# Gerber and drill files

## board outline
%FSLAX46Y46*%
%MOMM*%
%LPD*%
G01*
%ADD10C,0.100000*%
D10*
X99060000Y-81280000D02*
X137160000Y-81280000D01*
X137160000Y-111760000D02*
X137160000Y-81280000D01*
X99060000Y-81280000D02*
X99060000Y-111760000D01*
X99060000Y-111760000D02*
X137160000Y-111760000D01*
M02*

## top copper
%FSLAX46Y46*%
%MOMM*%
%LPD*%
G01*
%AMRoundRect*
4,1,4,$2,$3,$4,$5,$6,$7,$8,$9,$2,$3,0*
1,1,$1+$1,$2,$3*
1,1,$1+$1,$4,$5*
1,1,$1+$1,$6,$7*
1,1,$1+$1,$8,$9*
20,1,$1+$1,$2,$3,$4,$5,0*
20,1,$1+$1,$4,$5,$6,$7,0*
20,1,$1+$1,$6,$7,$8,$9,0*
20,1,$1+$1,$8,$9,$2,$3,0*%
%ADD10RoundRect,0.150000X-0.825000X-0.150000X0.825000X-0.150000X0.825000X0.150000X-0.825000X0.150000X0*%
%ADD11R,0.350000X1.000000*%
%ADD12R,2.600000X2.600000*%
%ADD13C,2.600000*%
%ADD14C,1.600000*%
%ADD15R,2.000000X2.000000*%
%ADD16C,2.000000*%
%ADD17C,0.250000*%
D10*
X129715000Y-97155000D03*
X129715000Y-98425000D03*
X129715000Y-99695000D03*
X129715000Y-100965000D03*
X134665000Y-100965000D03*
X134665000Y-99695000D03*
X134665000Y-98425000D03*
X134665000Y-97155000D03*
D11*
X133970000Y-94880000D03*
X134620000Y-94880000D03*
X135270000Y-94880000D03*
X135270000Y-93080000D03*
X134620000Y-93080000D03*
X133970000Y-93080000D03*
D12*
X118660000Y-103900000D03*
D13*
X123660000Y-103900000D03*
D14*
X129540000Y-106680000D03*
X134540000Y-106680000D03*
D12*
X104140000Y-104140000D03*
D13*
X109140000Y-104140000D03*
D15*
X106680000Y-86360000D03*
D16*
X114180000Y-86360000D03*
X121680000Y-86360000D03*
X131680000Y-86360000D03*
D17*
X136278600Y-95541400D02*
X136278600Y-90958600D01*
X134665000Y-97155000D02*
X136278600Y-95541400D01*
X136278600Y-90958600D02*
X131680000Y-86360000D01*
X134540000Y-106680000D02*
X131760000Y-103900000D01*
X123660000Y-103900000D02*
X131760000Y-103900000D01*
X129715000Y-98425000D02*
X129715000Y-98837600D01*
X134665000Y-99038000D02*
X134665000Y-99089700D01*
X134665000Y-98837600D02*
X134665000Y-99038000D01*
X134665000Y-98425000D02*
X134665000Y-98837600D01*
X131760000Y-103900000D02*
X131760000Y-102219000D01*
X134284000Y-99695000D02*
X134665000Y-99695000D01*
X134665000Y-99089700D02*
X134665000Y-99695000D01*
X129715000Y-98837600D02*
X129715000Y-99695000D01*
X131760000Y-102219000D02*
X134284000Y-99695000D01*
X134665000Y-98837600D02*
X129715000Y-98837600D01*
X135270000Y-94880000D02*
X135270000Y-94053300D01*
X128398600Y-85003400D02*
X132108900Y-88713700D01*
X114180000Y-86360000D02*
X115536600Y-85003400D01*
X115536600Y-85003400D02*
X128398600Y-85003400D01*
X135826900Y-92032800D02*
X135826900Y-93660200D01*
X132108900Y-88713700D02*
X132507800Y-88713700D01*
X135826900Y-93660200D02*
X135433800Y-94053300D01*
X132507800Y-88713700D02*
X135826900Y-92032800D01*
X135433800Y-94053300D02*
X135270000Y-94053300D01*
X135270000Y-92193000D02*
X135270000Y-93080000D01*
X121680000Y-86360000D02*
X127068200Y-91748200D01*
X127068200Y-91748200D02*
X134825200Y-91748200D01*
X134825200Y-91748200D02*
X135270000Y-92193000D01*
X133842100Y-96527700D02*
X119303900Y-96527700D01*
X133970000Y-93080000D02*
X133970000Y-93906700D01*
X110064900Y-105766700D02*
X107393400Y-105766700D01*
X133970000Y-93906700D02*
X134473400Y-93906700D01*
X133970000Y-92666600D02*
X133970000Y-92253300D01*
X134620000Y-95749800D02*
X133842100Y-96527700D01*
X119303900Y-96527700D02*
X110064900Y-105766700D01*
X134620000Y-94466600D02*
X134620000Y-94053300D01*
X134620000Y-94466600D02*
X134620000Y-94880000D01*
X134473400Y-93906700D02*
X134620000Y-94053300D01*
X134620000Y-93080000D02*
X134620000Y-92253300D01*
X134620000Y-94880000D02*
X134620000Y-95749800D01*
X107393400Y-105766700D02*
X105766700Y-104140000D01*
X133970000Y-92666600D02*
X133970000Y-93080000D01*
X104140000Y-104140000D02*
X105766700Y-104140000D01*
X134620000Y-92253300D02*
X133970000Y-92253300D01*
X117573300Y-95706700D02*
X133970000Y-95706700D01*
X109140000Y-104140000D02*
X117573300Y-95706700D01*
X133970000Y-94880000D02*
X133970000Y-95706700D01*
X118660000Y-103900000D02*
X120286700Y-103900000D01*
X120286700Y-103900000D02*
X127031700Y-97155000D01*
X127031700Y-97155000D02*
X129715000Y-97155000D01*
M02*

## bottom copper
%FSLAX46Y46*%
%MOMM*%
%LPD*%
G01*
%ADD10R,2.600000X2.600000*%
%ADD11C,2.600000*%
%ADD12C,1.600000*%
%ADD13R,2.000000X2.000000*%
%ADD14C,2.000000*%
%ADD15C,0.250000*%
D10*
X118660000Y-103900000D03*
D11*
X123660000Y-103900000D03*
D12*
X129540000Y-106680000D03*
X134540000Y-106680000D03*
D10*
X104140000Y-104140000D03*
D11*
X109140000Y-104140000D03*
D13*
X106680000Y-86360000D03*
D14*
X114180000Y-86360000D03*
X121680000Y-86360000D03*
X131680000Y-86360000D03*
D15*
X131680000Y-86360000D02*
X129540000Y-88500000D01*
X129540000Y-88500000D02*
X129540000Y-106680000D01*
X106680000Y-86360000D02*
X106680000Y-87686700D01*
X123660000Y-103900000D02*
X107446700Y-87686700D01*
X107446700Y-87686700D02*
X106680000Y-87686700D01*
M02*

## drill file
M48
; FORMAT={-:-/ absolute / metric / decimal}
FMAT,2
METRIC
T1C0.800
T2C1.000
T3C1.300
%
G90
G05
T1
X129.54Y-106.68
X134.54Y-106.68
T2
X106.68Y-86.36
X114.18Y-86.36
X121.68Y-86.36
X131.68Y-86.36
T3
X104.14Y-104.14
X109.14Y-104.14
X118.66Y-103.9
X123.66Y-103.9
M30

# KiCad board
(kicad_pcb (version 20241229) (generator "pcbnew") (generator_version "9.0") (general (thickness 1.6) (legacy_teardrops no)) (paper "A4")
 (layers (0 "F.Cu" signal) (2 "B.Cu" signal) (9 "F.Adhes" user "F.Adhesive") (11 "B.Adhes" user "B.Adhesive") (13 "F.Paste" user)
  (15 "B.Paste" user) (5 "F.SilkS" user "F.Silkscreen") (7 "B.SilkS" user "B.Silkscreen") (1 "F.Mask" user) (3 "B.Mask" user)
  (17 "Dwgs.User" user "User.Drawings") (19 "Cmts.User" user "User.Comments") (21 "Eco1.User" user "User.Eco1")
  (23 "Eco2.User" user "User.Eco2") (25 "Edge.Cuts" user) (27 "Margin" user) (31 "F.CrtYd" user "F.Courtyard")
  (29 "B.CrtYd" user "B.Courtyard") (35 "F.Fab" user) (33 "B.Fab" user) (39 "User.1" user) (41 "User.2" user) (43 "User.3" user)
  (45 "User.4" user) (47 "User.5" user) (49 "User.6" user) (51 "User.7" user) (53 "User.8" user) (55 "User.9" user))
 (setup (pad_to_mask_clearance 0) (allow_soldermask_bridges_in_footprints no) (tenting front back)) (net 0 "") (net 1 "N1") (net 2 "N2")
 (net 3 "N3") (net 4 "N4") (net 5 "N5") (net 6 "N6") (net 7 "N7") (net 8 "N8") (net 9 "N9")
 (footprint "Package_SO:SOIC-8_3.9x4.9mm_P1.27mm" (layer "F.Cu") (at 132.19 99.06)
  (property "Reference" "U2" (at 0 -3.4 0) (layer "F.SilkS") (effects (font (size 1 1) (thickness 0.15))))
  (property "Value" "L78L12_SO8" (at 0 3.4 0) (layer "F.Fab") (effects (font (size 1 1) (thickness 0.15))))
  (pad "1" smd roundrect (at -2.475 -1.905) (size 1.95 0.6) (layers "F.Cu" "F.Mask" "F.Paste") (roundrect_rratio 0.25) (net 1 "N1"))
  (pad "2" smd roundrect (at -2.475 -0.635) (size 1.95 0.6) (layers "F.Cu" "F.Mask" "F.Paste") (roundrect_rratio 0.25) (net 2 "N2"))
  (pad "3" smd roundrect (at -2.475 0.635) (size 1.95 0.6) (layers "F.Cu" "F.Mask" "F.Paste") (roundrect_rratio 0.25) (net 2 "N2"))
  (pad "4" smd roundrect (at -2.475 1.905) (size 1.95 0.6) (layers "F.Cu" "F.Mask" "F.Paste") (roundrect_rratio 0.25) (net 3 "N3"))
  (pad "5" smd roundrect (at 2.475 1.905) (size 1.95 0.6) (layers "F.Cu" "F.Mask" "F.Paste") (roundrect_rratio 0.25) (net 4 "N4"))
  (pad "6" smd roundrect (at 2.475 0.635) (size 1.95 0.6) (layers "F.Cu" "F.Mask" "F.Paste") (roundrect_rratio 0.25) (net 2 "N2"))
  (pad "7" smd roundrect (at 2.475 -0.635) (size 1.95 0.6) (layers "F.Cu" "F.Mask" "F.Paste") (roundrect_rratio 0.25) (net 2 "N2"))
  (pad "8" smd roundrect (at 2.475 -1.905) (size 1.95 0.6) (layers "F.Cu" "F.Mask" "F.Paste") (roundrect_rratio 0.25) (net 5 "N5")))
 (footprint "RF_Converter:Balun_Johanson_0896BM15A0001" (layer "F.Cu") (at 134.62 93.98 90)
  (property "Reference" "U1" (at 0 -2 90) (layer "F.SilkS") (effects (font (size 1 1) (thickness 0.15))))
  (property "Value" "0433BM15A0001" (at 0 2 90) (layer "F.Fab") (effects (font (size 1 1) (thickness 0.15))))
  (pad "1" smd rect (at -0.9 -0.65 90) (size 1 0.35) (layers "F.Cu" "F.Mask" "F.Paste") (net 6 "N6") (clearance 0.2))
  (pad "2" smd rect (at -0.9 0 90) (size 1 0.35) (layers "F.Cu" "F.Mask" "F.Paste") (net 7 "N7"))
  (pad "3" smd rect (at -0.9 0.65 90) (size 1 0.35) (layers "F.Cu" "F.Mask" "F.Paste") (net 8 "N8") (clearance 0.2))
  (pad "4" smd rect (at 0.9 0.65 90) (size 1 0.35) (layers "F.Cu" "F.Mask" "F.Paste") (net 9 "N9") (clearance 0.2))
  (pad "5" smd rect (at 0.9 0 90) (size 1 0.35) (layers "F.Cu" "F.Mask" "F.Paste") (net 7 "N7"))
  (pad "6" smd rect (at 0.9 -0.65 90) (size 1 0.35) (layers "F.Cu" "F.Mask" "F.Paste") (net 7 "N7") (clearance 0.2)))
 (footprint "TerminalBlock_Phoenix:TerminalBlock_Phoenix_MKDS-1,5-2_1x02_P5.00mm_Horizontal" (layer "F.Cu") (at 118.66 103.9)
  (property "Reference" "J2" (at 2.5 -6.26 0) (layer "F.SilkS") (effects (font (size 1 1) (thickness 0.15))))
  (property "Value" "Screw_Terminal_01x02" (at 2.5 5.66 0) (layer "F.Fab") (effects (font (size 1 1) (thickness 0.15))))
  (pad "1" thru_hole rect (at 0 0) (size 2.6 2.6) (drill 1.3) (layers "*.Cu" "*.Mask") (remove_unused_layers no) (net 1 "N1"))
  (pad "2" thru_hole circle (at 5 0) (size 2.6 2.6) (drill 1.3) (layers "*.Cu" "*.Mask") (remove_unused_layers no) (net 2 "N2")))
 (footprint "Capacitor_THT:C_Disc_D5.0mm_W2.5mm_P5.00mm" (layer "F.Cu") (at 129.54 106.68)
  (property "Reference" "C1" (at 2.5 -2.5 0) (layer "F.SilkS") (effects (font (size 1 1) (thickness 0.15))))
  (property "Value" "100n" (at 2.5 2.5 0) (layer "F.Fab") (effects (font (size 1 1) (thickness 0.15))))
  (pad "1" thru_hole circle (at 0 0) (size 1.6 1.6) (drill 0.8) (layers "*.Cu" "*.Mask") (remove_unused_layers no) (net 5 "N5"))
  (pad "2" thru_hole circle (at 5 0) (size 1.6 1.6) (drill 0.8) (layers "*.Cu" "*.Mask") (remove_unused_layers no) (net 2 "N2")))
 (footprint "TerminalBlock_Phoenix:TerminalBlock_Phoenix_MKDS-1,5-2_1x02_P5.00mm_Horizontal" (layer "F.Cu") (at 104.14 104.14)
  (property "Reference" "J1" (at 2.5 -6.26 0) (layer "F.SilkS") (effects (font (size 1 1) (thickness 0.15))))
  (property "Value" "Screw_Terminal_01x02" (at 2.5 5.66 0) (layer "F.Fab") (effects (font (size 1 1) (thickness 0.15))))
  (pad "1" thru_hole rect (at 0 0) (size 2.6 2.6) (drill 1.3) (layers "*.Cu" "*.Mask") (remove_unused_layers no) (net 7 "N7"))
  (pad "2" thru_hole circle (at 5 0) (size 2.6 2.6) (drill 1.3) (layers "*.Cu" "*.Mask") (remove_unused_layers no) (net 6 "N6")))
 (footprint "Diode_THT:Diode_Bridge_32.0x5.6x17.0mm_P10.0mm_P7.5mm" (layer "F.Cu") (at 106.68 86.36)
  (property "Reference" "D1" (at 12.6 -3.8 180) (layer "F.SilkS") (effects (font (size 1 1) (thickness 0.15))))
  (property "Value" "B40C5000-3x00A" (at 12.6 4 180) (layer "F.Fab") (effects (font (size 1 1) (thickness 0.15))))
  (pad "1" thru_hole rect (at 0 0) (size 2 2) (drill 1) (layers "*.Cu" "*.Mask") (remove_unused_layers no) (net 2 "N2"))
  (pad "2" thru_hole circle (at 7.5 0) (size 2 2) (drill 1) (layers "*.Cu" "*.Mask") (remove_unused_layers no) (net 8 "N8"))
  (pad "3" thru_hole circle (at 15 0) (size 2 2) (drill 1) (layers "*.Cu" "*.Mask") (remove_unused_layers no) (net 9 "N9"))
  (pad "4" thru_hole circle (at 25 0) (size 2 2) (drill 1) (layers "*.Cu" "*.Mask") (remove_unused_layers no) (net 5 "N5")))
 (gr_line (start 99.06 81.28) (end 137.16 81.28) (stroke (width 0.1) (type solid)) (layer "Edge.Cuts"))
 (gr_line (start 137.16 111.76) (end 137.16 81.28) (stroke (width 0.1) (type solid)) (layer "Edge.Cuts"))
 (gr_line (start 99.06 81.28) (end 99.06 111.76) (stroke (width 0.1) (type solid)) (layer "Edge.Cuts"))
 (gr_line (start 99.06 111.76) (end 137.16 111.76) (stroke (width 0.1) (type solid)) (layer "Edge.Cuts"))
 (segment (start 136.2786 95.5414) (end 136.2786 90.9586) (width 0.25) (layer "F.Cu") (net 5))
 (segment (start 134.665 97.155) (end 136.2786 95.5414) (width 0.25) (layer "F.Cu") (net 5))
 (segment (start 136.2786 90.9586) (end 131.68 86.36) (width 0.25) (layer "F.Cu") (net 5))
 (segment (start 131.68 86.36) (end 129.54 88.5) (width 0.25) (layer "B.Cu") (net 5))
 (segment (start 129.54 88.5) (end 129.54 106.68) (width 0.25) (layer "B.Cu") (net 5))
 (segment (start 134.54 106.68) (end 131.76 103.9) (width 0.25) (layer "F.Cu") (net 2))
 (segment (start 123.66 103.9) (end 131.76 103.9) (width 0.25) (layer "F.Cu") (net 2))
 (segment (start 129.715 98.425) (end 129.715 98.8376) (width 0.25) (layer "F.Cu") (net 2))
 (segment (start 134.665 99.038) (end 134.665 99.0897) (width 0.25) (layer "F.Cu") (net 2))
 (segment (start 134.665 98.8376) (end 134.665 99.038) (width 0.25) (layer "F.Cu") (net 2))
 (segment (start 134.665 98.425) (end 134.665 98.8376) (width 0.25) (layer "F.Cu") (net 2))
 (segment (start 131.76 103.9) (end 131.76 102.219) (width 0.25) (layer "F.Cu") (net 2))
 (segment (start 134.284 99.695) (end 134.665 99.695) (width 0.25) (layer "F.Cu") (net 2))
 (segment (start 134.665 99.0897) (end 134.665 99.695) (width 0.25) (layer "F.Cu") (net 2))
 (segment (start 129.715 98.8376) (end 129.715 99.695) (width 0.25) (layer "F.Cu") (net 2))
 (segment (start 131.76 102.219) (end 134.284 99.695) (width 0.25) (layer "F.Cu") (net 2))
 (segment (start 134.665 98.8376) (end 129.715 98.8376) (width 0.25) (layer "F.Cu") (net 2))
 (segment (start 106.68 86.36) (end 106.68 87.6867) (width 0.25) (layer "B.Cu") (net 2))
 (segment (start 123.66 103.9) (end 107.4467 87.6867) (width 0.25) (layer "B.Cu") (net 2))
 (segment (start 107.4467 87.6867) (end 106.68 87.6867) (width 0.25) (layer "B.Cu") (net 2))
 (segment (start 135.27 94.88) (end 135.27 94.0533) (width 0.25) (layer "F.Cu") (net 8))
 (segment (start 128.3986 85.0034) (end 132.1089 88.7137) (width 0.25) (layer "F.Cu") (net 8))
 (segment (start 114.18 86.36) (end 115.5366 85.0034) (width 0.25) (layer "F.Cu") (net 8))
 (segment (start 115.5366 85.0034) (end 128.3986 85.0034) (width 0.25) (layer "F.Cu") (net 8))
 (segment (start 135.8269 92.0328) (end 135.8269 93.6602) (width 0.25) (layer "F.Cu") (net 8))
 (segment (start 132.1089 88.7137) (end 132.5078 88.7137) (width 0.25) (layer "F.Cu") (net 8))
 (segment (start 135.8269 93.6602) (end 135.4338 94.0533) (width 0.25) (layer "F.Cu") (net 8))
 (segment (start 132.5078 88.7137) (end 135.8269 92.0328) (width 0.25) (layer "F.Cu") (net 8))
 (segment (start 135.4338 94.0533) (end 135.27 94.0533) (width 0.25) (layer "F.Cu") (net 8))
 (segment (start 135.27 92.193) (end 135.27 93.08) (width 0.25) (layer "F.Cu") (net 9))
 (segment (start 121.68 86.36) (end 127.0682 91.7482) (width 0.25) (layer "F.Cu") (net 9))
 (segment (start 127.0682 91.7482) (end 134.8252 91.7482) (width 0.25) (layer "F.Cu") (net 9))
 (segment (start 134.8252 91.7482) (end 135.27 92.193) (width 0.25) (layer "F.Cu") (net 9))
 (segment (start 133.8421 96.5277) (end 119.3039 96.5277) (width 0.25) (layer "F.Cu") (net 7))
 (segment (start 133.97 93.08) (end 133.97 93.9067) (width 0.25) (layer "F.Cu") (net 7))
 (segment (start 110.0649 105.7667) (end 107.3934 105.7667) (width 0.25) (layer "F.Cu") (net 7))
 (segment (start 133.97 93.9067) (end 134.4734 93.9067) (width 0.25) (layer "F.Cu") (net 7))
 (segment (start 133.97 92.6666) (end 133.97 92.2533) (width 0.25) (layer "F.Cu") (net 7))
 (segment (start 134.62 95.7498) (end 133.8421 96.5277) (width 0.25) (layer "F.Cu") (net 7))
 (segment (start 119.3039 96.5277) (end 110.0649 105.7667) (width 0.25) (layer "F.Cu") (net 7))
 (segment (start 134.62 94.4666) (end 134.62 94.0533) (width 0.25) (layer "F.Cu") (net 7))
 (segment (start 134.62 94.4666) (end 134.62 94.88) (width 0.25) (layer "F.Cu") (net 7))
 (segment (start 134.4734 93.9067) (end 134.62 94.0533) (width 0.25) (layer "F.Cu") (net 7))
 (segment (start 134.62 93.08) (end 134.62 92.2533) (width 0.25) (layer "F.Cu") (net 7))
 (segment (start 134.62 94.88) (end 134.62 95.7498) (width 0.25) (layer "F.Cu") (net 7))
 (segment (start 107.3934 105.7667) (end 105.7667 104.14) (width 0.25) (layer "F.Cu") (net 7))
 (segment (start 133.97 92.6666) (end 133.97 93.08) (width 0.25) (layer "F.Cu") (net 7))
 (segment (start 104.14 104.14) (end 105.7667 104.14) (width 0.25) (layer "F.Cu") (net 7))
 (segment (start 134.62 92.2533) (end 133.97 92.2533) (width 0.25) (layer "F.Cu") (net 7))
 (segment (start 117.5733 95.7067) (end 133.97 95.7067) (width 0.25) (layer "F.Cu") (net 6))
 (segment (start 109.14 104.14) (end 117.5733 95.7067) (width 0.25) (layer "F.Cu") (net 6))
 (segment (start 133.97 94.88) (end 133.97 95.7067) (width 0.25) (layer "F.Cu") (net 6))
 (segment (start 118.66 103.9) (end 120.2867 103.9) (width 0.25) (layer "F.Cu") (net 1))
 (segment (start 120.2867 103.9) (end 127.0317 97.155) (width 0.25) (layer "F.Cu") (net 1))
 (segment (start 127.0317 97.155) (end 129.715 97.155) (width 0.25) (layer "F.Cu") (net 1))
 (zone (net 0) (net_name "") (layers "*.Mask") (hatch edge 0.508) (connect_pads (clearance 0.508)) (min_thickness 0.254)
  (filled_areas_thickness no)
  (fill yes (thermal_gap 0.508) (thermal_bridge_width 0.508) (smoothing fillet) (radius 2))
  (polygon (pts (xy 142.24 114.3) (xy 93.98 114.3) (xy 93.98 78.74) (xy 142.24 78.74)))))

